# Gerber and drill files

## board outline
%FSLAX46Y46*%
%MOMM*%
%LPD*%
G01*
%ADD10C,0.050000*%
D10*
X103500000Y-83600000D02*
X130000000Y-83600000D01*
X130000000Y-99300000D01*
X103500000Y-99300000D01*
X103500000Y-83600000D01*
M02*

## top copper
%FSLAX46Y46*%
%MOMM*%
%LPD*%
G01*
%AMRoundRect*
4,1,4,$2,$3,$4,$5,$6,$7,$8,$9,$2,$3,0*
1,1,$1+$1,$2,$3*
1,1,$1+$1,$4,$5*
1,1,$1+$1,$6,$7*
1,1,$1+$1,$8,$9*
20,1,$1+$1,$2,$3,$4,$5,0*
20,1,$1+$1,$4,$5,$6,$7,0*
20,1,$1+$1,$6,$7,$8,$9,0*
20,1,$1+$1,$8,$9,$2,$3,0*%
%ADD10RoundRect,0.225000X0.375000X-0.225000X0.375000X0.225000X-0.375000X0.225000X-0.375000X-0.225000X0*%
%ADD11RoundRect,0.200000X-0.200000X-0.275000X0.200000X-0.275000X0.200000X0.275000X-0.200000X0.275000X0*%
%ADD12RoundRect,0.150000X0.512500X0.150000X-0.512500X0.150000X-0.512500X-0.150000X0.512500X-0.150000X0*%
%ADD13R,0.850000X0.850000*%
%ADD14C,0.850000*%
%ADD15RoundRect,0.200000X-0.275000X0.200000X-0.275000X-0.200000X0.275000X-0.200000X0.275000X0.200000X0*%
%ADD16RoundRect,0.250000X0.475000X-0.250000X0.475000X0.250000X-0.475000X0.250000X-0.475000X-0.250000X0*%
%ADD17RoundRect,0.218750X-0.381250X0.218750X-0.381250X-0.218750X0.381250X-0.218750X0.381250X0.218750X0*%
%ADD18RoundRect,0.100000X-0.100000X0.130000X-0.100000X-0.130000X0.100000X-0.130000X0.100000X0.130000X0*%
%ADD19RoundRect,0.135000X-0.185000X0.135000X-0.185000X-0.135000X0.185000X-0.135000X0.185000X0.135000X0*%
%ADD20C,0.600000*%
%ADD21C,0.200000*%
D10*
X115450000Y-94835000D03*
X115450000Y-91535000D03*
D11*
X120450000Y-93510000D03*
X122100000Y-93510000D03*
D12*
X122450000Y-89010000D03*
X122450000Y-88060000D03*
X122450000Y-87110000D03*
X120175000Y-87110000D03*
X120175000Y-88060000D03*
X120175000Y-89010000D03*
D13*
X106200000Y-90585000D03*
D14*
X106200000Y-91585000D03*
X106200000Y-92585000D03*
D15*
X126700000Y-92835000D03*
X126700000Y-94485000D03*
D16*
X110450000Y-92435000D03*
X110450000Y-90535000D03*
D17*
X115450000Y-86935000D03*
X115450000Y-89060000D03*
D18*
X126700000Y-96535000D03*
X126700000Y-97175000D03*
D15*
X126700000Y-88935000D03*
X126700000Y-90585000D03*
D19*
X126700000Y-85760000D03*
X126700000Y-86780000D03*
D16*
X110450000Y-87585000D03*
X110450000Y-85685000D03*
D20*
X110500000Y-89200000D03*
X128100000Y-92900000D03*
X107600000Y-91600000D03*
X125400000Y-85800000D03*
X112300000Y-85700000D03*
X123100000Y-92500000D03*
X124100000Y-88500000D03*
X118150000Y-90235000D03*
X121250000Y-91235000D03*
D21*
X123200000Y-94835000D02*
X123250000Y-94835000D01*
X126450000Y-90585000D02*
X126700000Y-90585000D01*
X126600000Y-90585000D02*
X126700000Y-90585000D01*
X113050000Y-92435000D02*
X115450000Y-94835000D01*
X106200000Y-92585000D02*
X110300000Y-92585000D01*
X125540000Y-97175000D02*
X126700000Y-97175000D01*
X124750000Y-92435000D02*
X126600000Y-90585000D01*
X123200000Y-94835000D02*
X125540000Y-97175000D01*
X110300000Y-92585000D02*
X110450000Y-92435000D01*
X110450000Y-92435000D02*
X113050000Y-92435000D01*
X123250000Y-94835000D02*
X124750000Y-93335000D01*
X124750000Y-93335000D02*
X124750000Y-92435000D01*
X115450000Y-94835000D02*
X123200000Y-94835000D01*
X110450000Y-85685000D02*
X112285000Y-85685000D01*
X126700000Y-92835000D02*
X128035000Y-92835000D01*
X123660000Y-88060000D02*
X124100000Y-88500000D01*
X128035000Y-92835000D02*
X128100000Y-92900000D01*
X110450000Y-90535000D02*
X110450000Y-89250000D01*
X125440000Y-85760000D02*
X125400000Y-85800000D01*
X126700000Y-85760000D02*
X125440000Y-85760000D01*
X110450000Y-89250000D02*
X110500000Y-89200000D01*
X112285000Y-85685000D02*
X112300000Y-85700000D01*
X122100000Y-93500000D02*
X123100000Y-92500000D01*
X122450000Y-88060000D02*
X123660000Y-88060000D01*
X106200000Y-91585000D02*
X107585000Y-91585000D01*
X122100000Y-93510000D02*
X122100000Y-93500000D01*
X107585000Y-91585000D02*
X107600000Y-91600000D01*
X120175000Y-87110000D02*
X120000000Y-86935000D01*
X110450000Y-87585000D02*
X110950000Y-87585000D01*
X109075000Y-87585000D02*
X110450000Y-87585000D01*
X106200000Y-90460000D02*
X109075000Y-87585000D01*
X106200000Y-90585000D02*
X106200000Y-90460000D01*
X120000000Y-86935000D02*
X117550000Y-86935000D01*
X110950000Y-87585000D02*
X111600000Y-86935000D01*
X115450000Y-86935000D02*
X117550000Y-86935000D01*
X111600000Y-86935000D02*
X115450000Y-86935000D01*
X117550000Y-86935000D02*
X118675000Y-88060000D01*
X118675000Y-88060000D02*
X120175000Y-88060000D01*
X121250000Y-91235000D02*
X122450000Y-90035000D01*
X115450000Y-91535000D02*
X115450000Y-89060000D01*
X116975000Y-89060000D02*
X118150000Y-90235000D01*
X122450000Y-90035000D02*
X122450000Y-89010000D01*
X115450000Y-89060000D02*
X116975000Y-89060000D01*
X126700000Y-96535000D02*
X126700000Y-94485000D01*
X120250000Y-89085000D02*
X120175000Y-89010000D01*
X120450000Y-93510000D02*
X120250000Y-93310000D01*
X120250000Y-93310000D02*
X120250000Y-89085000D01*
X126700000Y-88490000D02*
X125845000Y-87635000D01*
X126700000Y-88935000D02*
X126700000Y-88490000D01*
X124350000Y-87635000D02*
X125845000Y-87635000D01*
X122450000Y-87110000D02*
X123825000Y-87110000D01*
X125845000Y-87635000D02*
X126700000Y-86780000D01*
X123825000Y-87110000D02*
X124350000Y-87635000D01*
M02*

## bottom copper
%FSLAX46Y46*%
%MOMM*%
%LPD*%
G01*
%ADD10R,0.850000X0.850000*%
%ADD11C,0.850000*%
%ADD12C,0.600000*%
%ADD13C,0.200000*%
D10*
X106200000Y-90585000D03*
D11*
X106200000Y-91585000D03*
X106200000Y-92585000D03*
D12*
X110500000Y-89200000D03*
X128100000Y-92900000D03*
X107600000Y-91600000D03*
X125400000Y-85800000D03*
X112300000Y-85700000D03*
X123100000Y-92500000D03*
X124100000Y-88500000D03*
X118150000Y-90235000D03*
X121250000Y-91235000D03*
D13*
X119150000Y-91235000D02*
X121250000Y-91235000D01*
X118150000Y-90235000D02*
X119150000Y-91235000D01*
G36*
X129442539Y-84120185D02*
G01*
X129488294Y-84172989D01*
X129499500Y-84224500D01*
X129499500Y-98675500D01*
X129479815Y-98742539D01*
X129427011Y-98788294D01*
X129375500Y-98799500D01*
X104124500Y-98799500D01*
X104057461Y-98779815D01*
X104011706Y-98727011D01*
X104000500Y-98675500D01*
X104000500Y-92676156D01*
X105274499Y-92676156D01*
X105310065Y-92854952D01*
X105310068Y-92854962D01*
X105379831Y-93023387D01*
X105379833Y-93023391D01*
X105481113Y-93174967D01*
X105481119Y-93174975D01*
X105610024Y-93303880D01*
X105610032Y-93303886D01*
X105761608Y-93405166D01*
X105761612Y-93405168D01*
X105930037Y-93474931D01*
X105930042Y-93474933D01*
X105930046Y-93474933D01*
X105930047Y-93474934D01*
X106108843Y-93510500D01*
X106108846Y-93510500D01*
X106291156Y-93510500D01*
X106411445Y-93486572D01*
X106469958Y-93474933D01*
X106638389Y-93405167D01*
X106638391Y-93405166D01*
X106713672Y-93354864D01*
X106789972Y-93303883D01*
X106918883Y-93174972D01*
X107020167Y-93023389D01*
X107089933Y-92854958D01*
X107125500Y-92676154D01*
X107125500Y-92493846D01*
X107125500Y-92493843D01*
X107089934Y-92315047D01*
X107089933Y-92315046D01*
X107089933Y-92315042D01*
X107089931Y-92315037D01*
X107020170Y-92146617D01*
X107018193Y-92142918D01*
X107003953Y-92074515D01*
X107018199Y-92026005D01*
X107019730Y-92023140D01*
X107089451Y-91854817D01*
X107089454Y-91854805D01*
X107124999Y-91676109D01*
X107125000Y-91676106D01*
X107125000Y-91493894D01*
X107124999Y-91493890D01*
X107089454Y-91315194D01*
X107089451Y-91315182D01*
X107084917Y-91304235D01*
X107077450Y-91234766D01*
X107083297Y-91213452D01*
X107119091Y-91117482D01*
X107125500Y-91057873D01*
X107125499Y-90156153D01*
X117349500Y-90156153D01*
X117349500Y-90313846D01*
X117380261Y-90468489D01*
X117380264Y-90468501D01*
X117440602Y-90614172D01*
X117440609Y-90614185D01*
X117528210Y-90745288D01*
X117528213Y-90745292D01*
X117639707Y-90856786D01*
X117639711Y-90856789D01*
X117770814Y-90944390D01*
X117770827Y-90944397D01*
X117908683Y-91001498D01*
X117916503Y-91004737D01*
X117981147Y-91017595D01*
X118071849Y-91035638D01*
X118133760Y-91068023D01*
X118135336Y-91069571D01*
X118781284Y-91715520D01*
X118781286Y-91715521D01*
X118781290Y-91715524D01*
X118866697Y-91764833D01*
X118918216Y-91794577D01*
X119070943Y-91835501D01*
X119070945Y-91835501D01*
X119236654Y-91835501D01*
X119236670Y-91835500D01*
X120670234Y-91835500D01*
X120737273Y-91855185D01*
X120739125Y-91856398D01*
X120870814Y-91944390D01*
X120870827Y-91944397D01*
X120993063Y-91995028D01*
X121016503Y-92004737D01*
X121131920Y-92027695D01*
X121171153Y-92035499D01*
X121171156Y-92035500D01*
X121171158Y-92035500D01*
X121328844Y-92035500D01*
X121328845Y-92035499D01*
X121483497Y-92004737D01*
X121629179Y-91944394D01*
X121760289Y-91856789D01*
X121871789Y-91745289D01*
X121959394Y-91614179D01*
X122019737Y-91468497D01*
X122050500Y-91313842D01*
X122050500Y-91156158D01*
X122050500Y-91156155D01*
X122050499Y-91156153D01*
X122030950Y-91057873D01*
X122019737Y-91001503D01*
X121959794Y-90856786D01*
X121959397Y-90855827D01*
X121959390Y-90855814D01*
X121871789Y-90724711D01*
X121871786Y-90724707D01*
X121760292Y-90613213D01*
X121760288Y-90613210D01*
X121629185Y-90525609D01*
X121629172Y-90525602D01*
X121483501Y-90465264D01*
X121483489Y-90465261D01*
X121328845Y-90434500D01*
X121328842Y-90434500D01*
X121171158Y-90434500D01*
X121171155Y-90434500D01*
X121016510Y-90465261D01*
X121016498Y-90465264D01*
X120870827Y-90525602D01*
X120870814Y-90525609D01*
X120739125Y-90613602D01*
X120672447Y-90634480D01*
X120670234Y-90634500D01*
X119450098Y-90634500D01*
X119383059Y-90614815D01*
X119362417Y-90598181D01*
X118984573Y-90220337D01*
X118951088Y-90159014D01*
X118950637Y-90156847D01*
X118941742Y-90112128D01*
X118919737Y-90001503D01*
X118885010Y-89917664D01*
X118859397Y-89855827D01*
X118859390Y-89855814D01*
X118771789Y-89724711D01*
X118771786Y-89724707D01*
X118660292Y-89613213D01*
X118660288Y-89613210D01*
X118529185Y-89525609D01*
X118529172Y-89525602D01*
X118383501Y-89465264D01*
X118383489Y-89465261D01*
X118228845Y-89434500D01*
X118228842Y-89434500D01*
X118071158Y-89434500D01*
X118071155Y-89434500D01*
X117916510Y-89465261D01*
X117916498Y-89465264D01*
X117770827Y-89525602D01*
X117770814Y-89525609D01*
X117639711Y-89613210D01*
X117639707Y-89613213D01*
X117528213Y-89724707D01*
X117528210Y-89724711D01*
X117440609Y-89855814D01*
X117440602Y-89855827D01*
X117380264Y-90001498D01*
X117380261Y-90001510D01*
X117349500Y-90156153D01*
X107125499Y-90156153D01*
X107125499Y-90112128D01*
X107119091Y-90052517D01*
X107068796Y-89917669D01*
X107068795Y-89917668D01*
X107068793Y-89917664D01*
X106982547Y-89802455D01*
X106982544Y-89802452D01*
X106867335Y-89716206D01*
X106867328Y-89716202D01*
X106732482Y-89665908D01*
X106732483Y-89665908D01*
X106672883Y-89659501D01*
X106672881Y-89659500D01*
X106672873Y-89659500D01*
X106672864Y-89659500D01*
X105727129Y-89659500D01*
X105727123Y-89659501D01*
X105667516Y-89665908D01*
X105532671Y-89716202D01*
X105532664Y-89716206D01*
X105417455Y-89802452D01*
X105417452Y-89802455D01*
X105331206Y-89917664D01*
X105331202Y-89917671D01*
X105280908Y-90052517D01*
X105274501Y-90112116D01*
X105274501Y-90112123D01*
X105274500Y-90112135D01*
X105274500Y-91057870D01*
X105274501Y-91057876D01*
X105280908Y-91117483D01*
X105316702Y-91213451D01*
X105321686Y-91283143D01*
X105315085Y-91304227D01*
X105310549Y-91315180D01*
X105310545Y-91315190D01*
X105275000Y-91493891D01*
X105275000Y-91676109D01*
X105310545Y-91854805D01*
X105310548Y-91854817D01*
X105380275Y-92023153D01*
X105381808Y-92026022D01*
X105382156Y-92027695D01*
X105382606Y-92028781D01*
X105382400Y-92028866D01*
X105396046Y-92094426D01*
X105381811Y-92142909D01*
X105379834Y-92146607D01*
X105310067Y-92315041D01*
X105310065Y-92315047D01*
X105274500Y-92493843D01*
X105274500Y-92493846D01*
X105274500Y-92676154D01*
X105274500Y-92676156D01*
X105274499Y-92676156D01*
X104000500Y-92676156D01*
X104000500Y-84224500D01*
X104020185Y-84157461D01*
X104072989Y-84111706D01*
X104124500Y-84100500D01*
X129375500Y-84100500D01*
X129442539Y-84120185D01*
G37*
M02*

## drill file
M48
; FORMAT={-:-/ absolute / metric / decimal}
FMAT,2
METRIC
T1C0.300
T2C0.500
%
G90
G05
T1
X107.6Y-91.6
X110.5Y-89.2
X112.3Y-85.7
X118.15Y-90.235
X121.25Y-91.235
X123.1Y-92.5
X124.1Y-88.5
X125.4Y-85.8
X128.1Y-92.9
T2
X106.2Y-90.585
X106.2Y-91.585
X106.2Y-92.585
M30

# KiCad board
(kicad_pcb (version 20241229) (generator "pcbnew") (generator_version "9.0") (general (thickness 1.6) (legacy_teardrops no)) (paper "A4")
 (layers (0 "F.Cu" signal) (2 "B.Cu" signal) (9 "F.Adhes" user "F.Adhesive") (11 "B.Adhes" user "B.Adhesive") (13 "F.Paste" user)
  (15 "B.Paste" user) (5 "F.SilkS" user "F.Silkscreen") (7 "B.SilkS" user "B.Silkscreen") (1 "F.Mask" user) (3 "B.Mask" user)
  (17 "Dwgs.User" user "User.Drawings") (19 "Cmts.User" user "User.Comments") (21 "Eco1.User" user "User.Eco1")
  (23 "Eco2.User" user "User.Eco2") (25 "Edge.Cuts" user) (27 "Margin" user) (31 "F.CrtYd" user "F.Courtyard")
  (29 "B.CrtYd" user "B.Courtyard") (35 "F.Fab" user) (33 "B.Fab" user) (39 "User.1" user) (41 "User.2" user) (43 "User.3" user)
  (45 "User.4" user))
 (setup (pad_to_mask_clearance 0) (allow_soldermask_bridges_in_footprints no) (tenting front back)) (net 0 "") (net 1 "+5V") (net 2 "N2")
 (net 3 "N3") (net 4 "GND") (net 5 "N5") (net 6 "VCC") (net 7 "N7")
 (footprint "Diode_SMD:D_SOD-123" (layer "F.Cu") (at 115.45 93.185 90)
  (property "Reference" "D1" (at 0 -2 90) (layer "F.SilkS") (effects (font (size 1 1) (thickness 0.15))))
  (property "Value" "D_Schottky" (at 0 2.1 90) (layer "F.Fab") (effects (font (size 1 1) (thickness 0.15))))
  (pad "1" smd roundrect (at -1.65 0 90) (size 0.9 1.2) (layers "F.Cu" "F.Mask" "F.Paste") (roundrect_rratio 0.25) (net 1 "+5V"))
  (pad "2" smd roundrect (at 1.65 0 90) (size 0.9 1.2) (layers "F.Cu" "F.Mask" "F.Paste") (roundrect_rratio 0.25) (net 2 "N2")))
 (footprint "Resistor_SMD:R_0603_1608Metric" (layer "F.Cu") (at 121.275 93.51)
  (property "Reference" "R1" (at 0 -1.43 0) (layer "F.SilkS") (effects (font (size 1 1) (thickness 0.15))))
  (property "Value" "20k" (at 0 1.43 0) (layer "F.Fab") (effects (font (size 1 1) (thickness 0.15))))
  (pad "1" smd roundrect (at -0.825 0) (size 0.8 0.95) (layers "F.Cu" "F.Mask" "F.Paste") (roundrect_rratio 0.25) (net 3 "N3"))
  (pad "2" smd roundrect (at 0.825 0) (size 0.8 0.95) (layers "F.Cu" "F.Mask" "F.Paste") (roundrect_rratio 0.25) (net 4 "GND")))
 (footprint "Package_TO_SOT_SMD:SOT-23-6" (layer "F.Cu") (at 121.3125 88.06 180)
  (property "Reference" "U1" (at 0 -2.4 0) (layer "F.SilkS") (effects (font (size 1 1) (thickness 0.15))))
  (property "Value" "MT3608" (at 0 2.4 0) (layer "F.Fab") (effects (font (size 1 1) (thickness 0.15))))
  (pad "1" smd roundrect (at -1.1375 -0.95 180) (size 1.325 0.6) (layers "F.Cu" "F.Mask" "F.Paste") (roundrect_rratio 0.25) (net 2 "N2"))
  (pad "2" smd roundrect (at -1.1375 0 180) (size 1.325 0.6) (layers "F.Cu" "F.Mask" "F.Paste") (roundrect_rratio 0.25) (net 4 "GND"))
  (pad "3" smd roundrect (at -1.1375 0.95 180) (size 1.325 0.6) (layers "F.Cu" "F.Mask" "F.Paste") (roundrect_rratio 0.25) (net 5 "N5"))
  (pad "4" smd roundrect (at 1.1375 0.95 180) (size 1.325 0.6) (layers "F.Cu" "F.Mask" "F.Paste") (roundrect_rratio 0.25) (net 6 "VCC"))
  (pad "5" smd roundrect (at 1.1375 0 180) (size 1.325 0.6) (layers "F.Cu" "F.Mask" "F.Paste") (roundrect_rratio 0.25) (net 6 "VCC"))
  (pad "6" smd roundrect (at 1.1375 -0.95 180) (size 1.325 0.6) (layers "F.Cu" "F.Mask" "F.Paste") (roundrect_rratio 0.25) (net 3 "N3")))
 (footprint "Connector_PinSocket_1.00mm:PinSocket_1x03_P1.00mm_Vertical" (layer "F.Cu") (at 106.2 90.585)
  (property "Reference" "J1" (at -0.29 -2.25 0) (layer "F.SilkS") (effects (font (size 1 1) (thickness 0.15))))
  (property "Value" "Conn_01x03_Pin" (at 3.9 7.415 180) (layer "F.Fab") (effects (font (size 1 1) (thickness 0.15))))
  (pad "1" thru_hole rect (at 0 0) (size 0.85 0.85) (drill 0.5) (layers "*.Cu" "*.Mask") (remove_unused_layers no) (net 6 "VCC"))
  (pad "2" thru_hole circle (at 0 1) (size 0.85 0.85) (drill 0.5) (layers "*.Cu" "*.Mask") (remove_unused_layers no) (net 4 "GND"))
  (pad "3" thru_hole circle (at 0 2) (size 0.85 0.85) (drill 0.5) (layers "*.Cu" "*.Mask") (remove_unused_layers no) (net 1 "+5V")))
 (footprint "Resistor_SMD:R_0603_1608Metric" (layer "F.Cu") (at 126.7 93.66 -90)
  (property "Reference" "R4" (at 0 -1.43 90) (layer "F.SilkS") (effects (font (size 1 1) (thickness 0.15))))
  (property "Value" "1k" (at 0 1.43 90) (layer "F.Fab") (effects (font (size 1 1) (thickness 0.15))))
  (pad "1" smd roundrect (at -0.825 0 270) (size 0.8 0.95) (layers "F.Cu" "F.Mask" "F.Paste") (roundrect_rratio 0.25) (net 4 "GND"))
  (pad "2" smd roundrect (at 0.825 0 270) (size 0.8 0.95) (layers "F.Cu" "F.Mask" "F.Paste") (roundrect_rratio 0.25) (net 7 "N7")))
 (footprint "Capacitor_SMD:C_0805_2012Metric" (layer "F.Cu") (at 110.45 91.485 90)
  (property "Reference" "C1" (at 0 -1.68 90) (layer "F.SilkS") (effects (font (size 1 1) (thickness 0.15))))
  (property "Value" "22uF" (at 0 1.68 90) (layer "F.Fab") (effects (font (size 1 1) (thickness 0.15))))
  (pad "1" smd roundrect (at -0.95 0 90) (size 1 1.45) (layers "F.Cu" "F.Mask" "F.Paste") (roundrect_rratio 0.25) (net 1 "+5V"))
  (pad "2" smd roundrect (at 0.95 0 90) (size 1 1.45) (layers "F.Cu" "F.Mask" "F.Paste") (roundrect_rratio 0.25) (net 4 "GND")))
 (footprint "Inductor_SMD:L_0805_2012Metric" (layer "F.Cu") (at 115.45 87.9975 -90)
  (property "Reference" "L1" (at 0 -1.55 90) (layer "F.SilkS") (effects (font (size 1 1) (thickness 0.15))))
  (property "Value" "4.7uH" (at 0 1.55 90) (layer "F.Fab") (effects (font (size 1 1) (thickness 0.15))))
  (pad "1" smd roundrect (at -1.0625 0 270) (size 0.875 1.2) (layers "F.Cu" "F.Mask" "F.Paste") (roundrect_rratio 0.25) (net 6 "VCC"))
  (pad "2" smd roundrect (at 1.0625 0 270) (size 0.875 1.2) (layers "F.Cu" "F.Mask" "F.Paste") (roundrect_rratio 0.25) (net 2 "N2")))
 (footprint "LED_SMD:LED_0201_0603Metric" (layer "F.Cu") (at 126.7 96.855 -90)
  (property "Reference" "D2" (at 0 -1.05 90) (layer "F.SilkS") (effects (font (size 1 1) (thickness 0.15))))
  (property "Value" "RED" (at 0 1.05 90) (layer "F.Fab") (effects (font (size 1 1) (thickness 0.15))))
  (pad "" smd roundrect (at -0.345 0 270) (size 0.318 0.36) (layers "F.Paste") (roundrect_rratio 0.25))
  (pad "" smd roundrect (at 0.345 0 270) (size 0.318 0.36) (layers "F.Paste") (roundrect_rratio 0.25))
  (pad "1" smd roundrect (at -0.32 0 270) (size 0.46 0.4) (layers "F.Cu" "F.Mask") (roundrect_rratio 0.25) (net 7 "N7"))
  (pad "2" smd roundrect (at 0.32 0 270) (size 0.46 0.4) (layers "F.Cu" "F.Mask") (roundrect_rratio 0.25) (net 1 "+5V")))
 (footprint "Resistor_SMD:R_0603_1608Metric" (layer "F.Cu") (at 126.7 89.76 -90)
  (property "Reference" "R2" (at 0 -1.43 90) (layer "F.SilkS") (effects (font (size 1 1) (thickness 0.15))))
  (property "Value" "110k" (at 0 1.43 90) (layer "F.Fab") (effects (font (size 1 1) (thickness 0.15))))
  (pad "1" smd roundrect (at -0.825 0 270) (size 0.8 0.95) (layers "F.Cu" "F.Mask" "F.Paste") (roundrect_rratio 0.25) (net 5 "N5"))
  (pad "2" smd roundrect (at 0.825 0 270) (size 0.8 0.95) (layers "F.Cu" "F.Mask" "F.Paste") (roundrect_rratio 0.25) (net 1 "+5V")))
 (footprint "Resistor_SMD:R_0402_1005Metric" (layer "F.Cu") (at 126.7 86.27 -90)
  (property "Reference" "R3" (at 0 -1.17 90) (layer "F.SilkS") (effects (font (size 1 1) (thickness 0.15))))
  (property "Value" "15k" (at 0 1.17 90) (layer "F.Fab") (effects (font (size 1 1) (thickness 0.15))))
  (pad "1" smd roundrect (at -0.51 0 270) (size 0.54 0.64) (layers "F.Cu" "F.Mask" "F.Paste") (roundrect_rratio 0.25) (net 4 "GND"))
  (pad "2" smd roundrect (at 0.51 0 270) (size 0.54 0.64) (layers "F.Cu" "F.Mask" "F.Paste") (roundrect_rratio 0.25) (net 5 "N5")))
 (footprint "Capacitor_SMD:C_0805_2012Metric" (layer "F.Cu") (at 110.45 86.635 90)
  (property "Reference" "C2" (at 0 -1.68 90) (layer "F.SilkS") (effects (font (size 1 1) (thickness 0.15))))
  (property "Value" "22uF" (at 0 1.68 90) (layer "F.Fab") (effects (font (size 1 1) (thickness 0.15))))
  (pad "1" smd roundrect (at -0.95 0 90) (size 1 1.45) (layers "F.Cu" "F.Mask" "F.Paste") (roundrect_rratio 0.25) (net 6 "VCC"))
  (pad "2" smd roundrect (at 0.95 0 90) (size 1 1.45) (layers "F.Cu" "F.Mask" "F.Paste") (roundrect_rratio 0.25) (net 4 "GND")))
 (gr_rect (start 103.5 83.6) (end 130 99.3) (stroke (width 0.05) (type default)) (fill no) (layer "Edge.Cuts"))
 (segment (start 123.2 94.835) (end 123.25 94.835) (width 0.2) (layer "F.Cu") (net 1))
 (segment (start 126.45 90.585) (end 126.7 90.585) (width 0.2) (layer "F.Cu") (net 1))
 (segment (start 126.6 90.585) (end 126.7 90.585) (width 0.2) (layer "F.Cu") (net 1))
 (segment (start 113.05 92.435) (end 115.45 94.835) (width 0.2) (layer "F.Cu") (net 1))
 (segment (start 106.2 92.585) (end 110.3 92.585) (width 0.2) (layer "F.Cu") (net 1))
 (segment (start 125.54 97.175) (end 126.7 97.175) (width 0.2) (layer "F.Cu") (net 1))
 (segment (start 124.75 92.435) (end 126.6 90.585) (width 0.2) (layer "F.Cu") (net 1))
 (segment (start 123.2 94.835) (end 125.54 97.175) (width 0.2) (layer "F.Cu") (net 1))
 (segment (start 110.3 92.585) (end 110.45 92.435) (width 0.2) (layer "F.Cu") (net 1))
 (segment (start 110.45 92.435) (end 113.05 92.435) (width 0.2) (layer "F.Cu") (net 1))
 (segment (start 123.25 94.835) (end 124.75 93.335) (width 0.2) (layer "F.Cu") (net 1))
 (segment (start 124.75 93.335) (end 124.75 92.435) (width 0.2) (layer "F.Cu") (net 1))
 (segment (start 115.45 94.835) (end 123.2 94.835) (width 0.2) (layer "F.Cu") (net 1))
 (segment (start 110.45 85.685) (end 112.285 85.685) (width 0.2) (layer "F.Cu") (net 4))
 (segment (start 126.7 92.835) (end 128.035 92.835) (width 0.2) (layer "F.Cu") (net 4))
 (segment (start 123.66 88.06) (end 124.1 88.5) (width 0.2) (layer "F.Cu") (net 4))
 (segment (start 128.035 92.835) (end 128.1 92.9) (width 0.2) (layer "F.Cu") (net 4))
 (segment (start 110.45 90.535) (end 110.45 89.25) (width 0.2) (layer "F.Cu") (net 4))
 (segment (start 125.44 85.76) (end 125.4 85.8) (width 0.2) (layer "F.Cu") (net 4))
 (segment (start 126.7 85.76) (end 125.44 85.76) (width 0.2) (layer "F.Cu") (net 4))
 (segment (start 110.45 89.25) (end 110.5 89.2) (width 0.2) (layer "F.Cu") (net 4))
 (segment (start 112.285 85.685) (end 112.3 85.7) (width 0.2) (layer "F.Cu") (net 4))
 (segment (start 122.1 93.5) (end 123.1 92.5) (width 0.2) (layer "F.Cu") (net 4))
 (segment (start 122.45 88.06) (end 123.66 88.06) (width 0.2) (layer "F.Cu") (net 4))
 (segment (start 106.2 91.585) (end 107.585 91.585) (width 0.2) (layer "F.Cu") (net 4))
 (segment (start 122.1 93.51) (end 122.1 93.5) (width 0.2) (layer "F.Cu") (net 4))
 (segment (start 107.585 91.585) (end 107.6 91.6) (width 0.2) (layer "F.Cu") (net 4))
 (via (at 110.5 89.2) (size 0.6) (drill 0.3) (layers "F.Cu" "B.Cu") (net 4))
 (via (at 128.1 92.9) (size 0.6) (drill 0.3) (layers "F.Cu" "B.Cu") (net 4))
 (via (at 107.6 91.6) (size 0.6) (drill 0.3) (layers "F.Cu" "B.Cu") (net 4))
 (via (at 125.4 85.8) (size 0.6) (drill 0.3) (layers "F.Cu" "B.Cu") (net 4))
 (via (at 112.3 85.7) (size 0.6) (drill 0.3) (layers "F.Cu" "B.Cu") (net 4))
 (via (at 123.1 92.5) (size 0.6) (drill 0.3) (layers "F.Cu" "B.Cu") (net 4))
 (via (at 124.1 88.5) (size 0.6) (drill 0.3) (layers "F.Cu" "B.Cu") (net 4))
 (segment (start 120.175 87.11) (end 120 86.935) (width 0.2) (layer "F.Cu") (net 6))
 (segment (start 110.45 87.585) (end 110.95 87.585) (width 0.2) (layer "F.Cu") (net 6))
 (segment (start 109.075 87.585) (end 110.45 87.585) (width 0.2) (layer "F.Cu") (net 6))
 (segment (start 106.2 90.46) (end 109.075 87.585) (width 0.2) (layer "F.Cu") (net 6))
 (segment (start 106.2 90.585) (end 106.2 90.46) (width 0.2) (layer "F.Cu") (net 6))
 (segment (start 120 86.935) (end 117.55 86.935) (width 0.2) (layer "F.Cu") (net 6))
 (segment (start 110.95 87.585) (end 111.6 86.935) (width 0.2) (layer "F.Cu") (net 6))
 (segment (start 115.45 86.935) (end 117.55 86.935) (width 0.2) (layer "F.Cu") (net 6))
 (segment (start 111.6 86.935) (end 115.45 86.935) (width 0.2) (layer "F.Cu") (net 6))
 (segment (start 117.55 86.935) (end 118.675 88.06) (width 0.2) (layer "F.Cu") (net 6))
 (segment (start 118.675 88.06) (end 120.175 88.06) (width 0.2) (layer "F.Cu") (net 6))
 (segment (start 121.25 91.235) (end 122.45 90.035) (width 0.2) (layer "F.Cu") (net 2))
 (segment (start 115.45 91.535) (end 115.45 89.06) (width 0.2) (layer "F.Cu") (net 2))
 (segment (start 116.975 89.06) (end 118.15 90.235) (width 0.2) (layer "F.Cu") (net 2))
 (segment (start 122.45 90.035) (end 122.45 89.01) (width 0.2) (layer "F.Cu") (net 2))
 (segment (start 115.45 89.06) (end 116.975 89.06) (width 0.2) (layer "F.Cu") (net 2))
 (via (at 118.15 90.235) (size 0.6) (drill 0.3) (layers "F.Cu" "B.Cu") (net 2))
 (via (at 121.25 91.235) (size 0.6) (drill 0.3) (layers "F.Cu" "B.Cu") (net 2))
 (segment (start 119.15 91.235) (end 121.25 91.235) (width 0.2) (layer "B.Cu") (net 2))
 (segment (start 118.15 90.235) (end 119.15 91.235) (width 0.2) (layer "B.Cu") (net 2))
 (segment (start 126.7 96.535) (end 126.7 94.485) (width 0.2) (layer "F.Cu") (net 7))
 (segment (start 120.25 89.085) (end 120.175 89.01) (width 0.2) (layer "F.Cu") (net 3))
 (segment (start 120.45 93.51) (end 120.25 93.31) (width 0.2) (layer "F.Cu") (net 3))
 (segment (start 120.25 93.31) (end 120.25 89.085) (width 0.2) (layer "F.Cu") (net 3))
 (segment (start 126.7 88.49) (end 125.845 87.635) (width 0.2) (layer "F.Cu") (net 5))
 (segment (start 126.7 88.935) (end 126.7 88.49) (width 0.2) (layer "F.Cu") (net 5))
 (segment (start 124.35 87.635) (end 125.845 87.635) (width 0.2) (layer "F.Cu") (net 5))
 (segment (start 122.45 87.11) (end 123.825 87.11) (width 0.2) (layer "F.Cu") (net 5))
 (segment (start 125.845 87.635) (end 126.7 86.78) (width 0.2) (layer "F.Cu") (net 5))
 (segment (start 123.825 87.11) (end 124.35 87.635) (width 0.2) (layer "F.Cu") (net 5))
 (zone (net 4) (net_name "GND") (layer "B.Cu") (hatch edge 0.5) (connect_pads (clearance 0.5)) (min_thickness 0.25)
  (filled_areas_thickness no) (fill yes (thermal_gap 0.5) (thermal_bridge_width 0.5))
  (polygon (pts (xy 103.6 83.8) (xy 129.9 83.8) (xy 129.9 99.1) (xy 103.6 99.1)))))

